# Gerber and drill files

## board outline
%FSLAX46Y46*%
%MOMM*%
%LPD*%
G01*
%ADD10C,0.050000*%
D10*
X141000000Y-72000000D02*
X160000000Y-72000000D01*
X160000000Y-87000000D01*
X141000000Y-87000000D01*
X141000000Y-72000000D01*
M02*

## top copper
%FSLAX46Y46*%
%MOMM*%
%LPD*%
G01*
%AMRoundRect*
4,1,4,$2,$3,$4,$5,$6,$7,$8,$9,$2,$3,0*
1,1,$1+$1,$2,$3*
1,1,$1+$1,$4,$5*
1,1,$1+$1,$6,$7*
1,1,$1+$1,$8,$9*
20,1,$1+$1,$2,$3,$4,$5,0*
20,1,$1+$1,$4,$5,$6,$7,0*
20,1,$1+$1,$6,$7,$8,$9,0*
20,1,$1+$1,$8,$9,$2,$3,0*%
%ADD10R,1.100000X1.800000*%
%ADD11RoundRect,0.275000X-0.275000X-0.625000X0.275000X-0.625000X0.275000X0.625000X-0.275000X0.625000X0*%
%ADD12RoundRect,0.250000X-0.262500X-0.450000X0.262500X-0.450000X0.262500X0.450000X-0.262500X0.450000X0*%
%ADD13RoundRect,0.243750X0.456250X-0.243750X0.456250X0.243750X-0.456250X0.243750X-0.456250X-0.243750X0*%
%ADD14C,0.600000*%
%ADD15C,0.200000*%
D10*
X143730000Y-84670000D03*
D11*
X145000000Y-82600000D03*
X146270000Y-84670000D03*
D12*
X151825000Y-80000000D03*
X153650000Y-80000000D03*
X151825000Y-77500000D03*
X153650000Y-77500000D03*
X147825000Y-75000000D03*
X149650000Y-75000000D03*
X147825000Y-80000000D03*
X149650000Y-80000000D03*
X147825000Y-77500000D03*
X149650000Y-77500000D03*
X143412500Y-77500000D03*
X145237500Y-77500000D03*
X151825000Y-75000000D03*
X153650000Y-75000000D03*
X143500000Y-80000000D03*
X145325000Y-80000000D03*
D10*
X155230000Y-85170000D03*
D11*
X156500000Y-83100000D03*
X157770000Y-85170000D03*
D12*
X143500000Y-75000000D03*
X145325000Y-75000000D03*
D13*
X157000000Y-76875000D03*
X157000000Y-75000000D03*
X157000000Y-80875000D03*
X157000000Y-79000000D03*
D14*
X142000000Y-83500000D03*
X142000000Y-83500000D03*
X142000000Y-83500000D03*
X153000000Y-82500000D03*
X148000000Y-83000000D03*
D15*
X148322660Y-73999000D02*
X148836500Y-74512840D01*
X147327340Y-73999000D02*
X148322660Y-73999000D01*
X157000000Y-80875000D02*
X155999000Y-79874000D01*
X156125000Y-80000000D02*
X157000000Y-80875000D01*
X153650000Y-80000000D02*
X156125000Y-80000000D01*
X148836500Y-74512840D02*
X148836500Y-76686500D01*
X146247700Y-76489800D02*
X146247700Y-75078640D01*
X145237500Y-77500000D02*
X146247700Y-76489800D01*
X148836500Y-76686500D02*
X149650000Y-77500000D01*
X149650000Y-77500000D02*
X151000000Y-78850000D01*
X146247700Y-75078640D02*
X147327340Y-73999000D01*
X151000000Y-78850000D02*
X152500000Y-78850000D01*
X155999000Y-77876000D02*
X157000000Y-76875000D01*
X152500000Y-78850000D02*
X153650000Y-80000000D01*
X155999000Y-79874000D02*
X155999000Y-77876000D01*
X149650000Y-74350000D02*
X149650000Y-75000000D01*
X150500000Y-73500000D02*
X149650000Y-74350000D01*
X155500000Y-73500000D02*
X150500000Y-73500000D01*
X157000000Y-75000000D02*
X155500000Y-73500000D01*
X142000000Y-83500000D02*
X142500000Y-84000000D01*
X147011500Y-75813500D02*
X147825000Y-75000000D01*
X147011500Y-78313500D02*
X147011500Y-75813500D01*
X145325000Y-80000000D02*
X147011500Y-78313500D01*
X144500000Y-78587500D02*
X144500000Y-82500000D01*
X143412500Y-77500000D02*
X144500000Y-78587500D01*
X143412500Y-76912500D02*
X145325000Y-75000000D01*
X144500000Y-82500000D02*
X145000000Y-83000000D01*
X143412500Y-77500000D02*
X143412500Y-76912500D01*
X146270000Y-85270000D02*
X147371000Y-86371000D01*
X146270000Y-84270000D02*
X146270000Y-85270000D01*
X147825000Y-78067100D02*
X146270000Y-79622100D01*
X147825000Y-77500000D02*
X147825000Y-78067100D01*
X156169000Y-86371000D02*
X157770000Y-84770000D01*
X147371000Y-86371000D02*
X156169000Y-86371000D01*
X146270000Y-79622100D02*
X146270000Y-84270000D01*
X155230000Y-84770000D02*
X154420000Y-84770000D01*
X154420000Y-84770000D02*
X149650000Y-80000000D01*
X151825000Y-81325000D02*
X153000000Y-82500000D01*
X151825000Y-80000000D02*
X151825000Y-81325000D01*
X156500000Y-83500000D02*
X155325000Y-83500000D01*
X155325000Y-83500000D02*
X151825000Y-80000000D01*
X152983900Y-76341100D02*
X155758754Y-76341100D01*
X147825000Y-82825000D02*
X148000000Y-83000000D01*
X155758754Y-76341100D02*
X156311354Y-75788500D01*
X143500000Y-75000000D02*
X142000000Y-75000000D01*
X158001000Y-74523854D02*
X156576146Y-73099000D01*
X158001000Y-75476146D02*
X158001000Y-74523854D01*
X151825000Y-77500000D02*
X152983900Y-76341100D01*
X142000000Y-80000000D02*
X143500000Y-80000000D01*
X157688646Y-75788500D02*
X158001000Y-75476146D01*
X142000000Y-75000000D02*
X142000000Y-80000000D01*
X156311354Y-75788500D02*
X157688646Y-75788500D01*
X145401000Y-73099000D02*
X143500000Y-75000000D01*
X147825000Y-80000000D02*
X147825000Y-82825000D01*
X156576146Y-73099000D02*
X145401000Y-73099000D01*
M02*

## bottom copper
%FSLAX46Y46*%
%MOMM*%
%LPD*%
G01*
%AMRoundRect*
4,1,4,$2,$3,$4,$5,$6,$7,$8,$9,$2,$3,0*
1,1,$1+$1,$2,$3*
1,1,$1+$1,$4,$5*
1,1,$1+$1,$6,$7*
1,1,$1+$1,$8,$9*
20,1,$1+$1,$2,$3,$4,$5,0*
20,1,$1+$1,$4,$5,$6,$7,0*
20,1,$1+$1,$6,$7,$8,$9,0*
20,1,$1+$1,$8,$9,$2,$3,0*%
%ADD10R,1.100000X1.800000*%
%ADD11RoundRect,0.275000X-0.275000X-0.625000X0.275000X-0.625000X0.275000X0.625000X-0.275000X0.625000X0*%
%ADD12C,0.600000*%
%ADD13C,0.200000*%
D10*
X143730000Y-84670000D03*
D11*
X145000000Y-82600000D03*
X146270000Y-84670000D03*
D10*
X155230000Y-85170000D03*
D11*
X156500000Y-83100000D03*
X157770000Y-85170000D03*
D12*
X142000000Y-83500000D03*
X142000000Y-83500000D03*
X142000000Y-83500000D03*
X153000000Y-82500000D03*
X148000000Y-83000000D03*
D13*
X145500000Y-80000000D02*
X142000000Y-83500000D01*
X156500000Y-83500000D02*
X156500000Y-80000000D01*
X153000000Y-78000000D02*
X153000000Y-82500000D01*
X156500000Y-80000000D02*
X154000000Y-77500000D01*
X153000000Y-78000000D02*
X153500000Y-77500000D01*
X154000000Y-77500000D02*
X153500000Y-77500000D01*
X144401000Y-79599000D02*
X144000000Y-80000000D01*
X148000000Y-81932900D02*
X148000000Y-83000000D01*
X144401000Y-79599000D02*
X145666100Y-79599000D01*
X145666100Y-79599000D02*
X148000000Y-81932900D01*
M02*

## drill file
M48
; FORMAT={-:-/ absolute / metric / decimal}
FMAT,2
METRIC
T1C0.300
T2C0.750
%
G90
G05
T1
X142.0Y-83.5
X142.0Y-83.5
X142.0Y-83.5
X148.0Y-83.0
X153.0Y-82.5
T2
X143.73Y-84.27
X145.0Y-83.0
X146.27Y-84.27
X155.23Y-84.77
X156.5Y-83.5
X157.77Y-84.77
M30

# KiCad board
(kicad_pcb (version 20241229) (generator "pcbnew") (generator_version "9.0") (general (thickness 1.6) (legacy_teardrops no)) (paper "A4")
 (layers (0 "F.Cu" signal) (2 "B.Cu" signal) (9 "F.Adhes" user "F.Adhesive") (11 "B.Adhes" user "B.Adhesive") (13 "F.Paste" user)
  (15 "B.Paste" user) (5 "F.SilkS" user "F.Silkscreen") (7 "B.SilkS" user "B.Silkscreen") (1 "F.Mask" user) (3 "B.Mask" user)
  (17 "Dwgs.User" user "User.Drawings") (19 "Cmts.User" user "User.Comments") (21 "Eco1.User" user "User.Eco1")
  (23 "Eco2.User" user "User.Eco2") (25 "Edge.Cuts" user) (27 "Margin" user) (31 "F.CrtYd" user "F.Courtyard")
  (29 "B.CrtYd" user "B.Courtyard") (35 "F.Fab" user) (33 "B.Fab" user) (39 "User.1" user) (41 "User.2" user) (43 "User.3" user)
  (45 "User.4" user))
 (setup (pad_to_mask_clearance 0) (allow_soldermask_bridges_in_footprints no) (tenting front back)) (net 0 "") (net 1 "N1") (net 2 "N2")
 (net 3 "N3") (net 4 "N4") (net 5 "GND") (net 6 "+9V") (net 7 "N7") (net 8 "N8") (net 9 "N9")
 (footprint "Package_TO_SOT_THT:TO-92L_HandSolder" (layer "F.Cu") (at 143.73 84.27)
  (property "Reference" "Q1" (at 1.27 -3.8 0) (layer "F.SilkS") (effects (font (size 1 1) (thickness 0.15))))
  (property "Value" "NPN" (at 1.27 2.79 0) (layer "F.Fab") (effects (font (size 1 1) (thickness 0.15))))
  (pad "1" thru_hole rect (at 0 0) (size 1.1 1.8) (drill 0.75 (offset 0 0.4)) (layers "*.Cu" "*.Mask") (remove_unused_layers no)
   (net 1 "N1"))
  (pad "2" thru_hole roundrect (at 1.27 -1.27) (size 1.1 1.8) (drill 0.75 (offset 0 -0.4)) (layers "*.Cu" "*.Mask")
   (remove_unused_layers no) (roundrect_rratio 0.25) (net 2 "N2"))
  (pad "3" thru_hole roundrect (at 2.54 0) (size 1.1 1.8) (drill 0.75 (offset 0 0.4)) (layers "*.Cu" "*.Mask") (remove_unused_layers no)
   (roundrect_rratio 0.25) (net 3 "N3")))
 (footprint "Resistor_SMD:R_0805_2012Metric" (layer "F.Cu") (at 152.7375 80)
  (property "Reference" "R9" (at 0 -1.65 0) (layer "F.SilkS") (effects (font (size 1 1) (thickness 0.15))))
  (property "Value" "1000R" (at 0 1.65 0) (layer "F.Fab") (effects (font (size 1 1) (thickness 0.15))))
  (pad "1" smd roundrect (at -0.9125 0) (size 1.025 1.4) (layers "F.Cu" "F.Mask" "F.Paste") (roundrect_rratio 0.243902) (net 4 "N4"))
  (pad "2" smd roundrect (at 0.9125 0) (size 1.025 1.4) (layers "F.Cu" "F.Mask" "F.Paste") (roundrect_rratio 0.243902) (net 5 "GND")))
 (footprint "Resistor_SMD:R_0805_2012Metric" (layer "F.Cu") (at 152.7375 77.5)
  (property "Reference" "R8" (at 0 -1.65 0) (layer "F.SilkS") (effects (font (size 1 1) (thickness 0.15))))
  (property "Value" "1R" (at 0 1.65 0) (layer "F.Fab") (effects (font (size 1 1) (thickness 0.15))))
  (pad "1" smd roundrect (at -0.9125 0) (size 1.025 1.4) (layers "F.Cu" "F.Mask" "F.Paste") (roundrect_rratio 0.243902) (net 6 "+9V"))
  (pad "2" smd roundrect (at 0.9125 0) (size 1.025 1.4) (layers "F.Cu" "F.Mask" "F.Paste") (roundrect_rratio 0.243902) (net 4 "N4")))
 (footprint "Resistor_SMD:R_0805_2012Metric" (layer "F.Cu") (at 148.7375 75)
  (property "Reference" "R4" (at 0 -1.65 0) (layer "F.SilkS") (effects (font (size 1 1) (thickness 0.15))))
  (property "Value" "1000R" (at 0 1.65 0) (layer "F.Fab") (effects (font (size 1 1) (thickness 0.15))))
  (pad "1" smd roundrect (at -0.9125 0) (size 1.025 1.4) (layers "F.Cu" "F.Mask" "F.Paste") (roundrect_rratio 0.243902) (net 1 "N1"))
  (pad "2" smd roundrect (at 0.9125 0) (size 1.025 1.4) (layers "F.Cu" "F.Mask" "F.Paste") (roundrect_rratio 0.243902) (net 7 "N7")))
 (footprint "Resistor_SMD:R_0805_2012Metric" (layer "F.Cu") (at 148.7375 80)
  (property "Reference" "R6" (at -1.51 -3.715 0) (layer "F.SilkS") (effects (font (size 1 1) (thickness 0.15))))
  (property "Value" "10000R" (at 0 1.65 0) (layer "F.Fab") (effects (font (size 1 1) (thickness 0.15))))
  (pad "1" smd roundrect (at -0.9125 0) (size 1.025 1.4) (layers "F.Cu" "F.Mask" "F.Paste") (roundrect_rratio 0.243902) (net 6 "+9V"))
  (pad "2" smd roundrect (at 0.9125 0) (size 1.025 1.4) (layers "F.Cu" "F.Mask" "F.Paste") (roundrect_rratio 0.243902) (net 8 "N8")))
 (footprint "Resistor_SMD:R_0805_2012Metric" (layer "F.Cu") (at 148.7375 77.5)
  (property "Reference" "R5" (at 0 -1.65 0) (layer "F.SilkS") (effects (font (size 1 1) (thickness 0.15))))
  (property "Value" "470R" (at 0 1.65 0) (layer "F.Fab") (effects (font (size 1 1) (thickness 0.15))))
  (pad "1" smd roundrect (at -0.9125 0) (size 1.025 1.4) (layers "F.Cu" "F.Mask" "F.Paste") (roundrect_rratio 0.243902) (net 3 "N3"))
  (pad "2" smd roundrect (at 0.9125 0) (size 1.025 1.4) (layers "F.Cu" "F.Mask" "F.Paste") (roundrect_rratio 0.243902) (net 5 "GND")))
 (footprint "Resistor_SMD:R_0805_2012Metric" (layer "F.Cu") (at 144.325 77.5)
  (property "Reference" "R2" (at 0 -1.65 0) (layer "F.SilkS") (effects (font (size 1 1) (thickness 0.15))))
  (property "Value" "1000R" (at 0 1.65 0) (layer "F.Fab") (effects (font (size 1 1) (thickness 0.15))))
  (pad "1" smd roundrect (at -0.9125 0) (size 1.025 1.4) (layers "F.Cu" "F.Mask" "F.Paste") (roundrect_rratio 0.243902) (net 2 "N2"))
  (pad "2" smd roundrect (at 0.9125 0) (size 1.025 1.4) (layers "F.Cu" "F.Mask" "F.Paste") (roundrect_rratio 0.243902) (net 5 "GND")))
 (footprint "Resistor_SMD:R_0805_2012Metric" (layer "F.Cu") (at 152.7375 75)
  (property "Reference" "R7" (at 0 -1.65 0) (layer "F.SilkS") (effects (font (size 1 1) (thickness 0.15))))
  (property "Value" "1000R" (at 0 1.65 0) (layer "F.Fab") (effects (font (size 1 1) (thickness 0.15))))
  (pad "1" smd roundrect (at -0.9125 0) (size 1.025 1.4) (layers "F.Cu" "F.Mask" "F.Paste") (roundrect_rratio 0.243902) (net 8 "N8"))
  (pad "2" smd roundrect (at 0.9125 0) (size 1.025 1.4) (layers "F.Cu" "F.Mask" "F.Paste") (roundrect_rratio 0.243902) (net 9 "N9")))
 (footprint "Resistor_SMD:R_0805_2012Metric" (layer "F.Cu") (at 144.4125 80)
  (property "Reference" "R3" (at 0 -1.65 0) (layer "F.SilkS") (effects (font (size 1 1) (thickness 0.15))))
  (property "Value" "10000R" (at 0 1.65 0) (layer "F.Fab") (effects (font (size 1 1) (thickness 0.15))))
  (pad "1" smd roundrect (at -0.9125 0) (size 1.025 1.4) (layers "F.Cu" "F.Mask" "F.Paste") (roundrect_rratio 0.243902) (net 6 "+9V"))
  (pad "2" smd roundrect (at 0.9125 0) (size 1.025 1.4) (layers "F.Cu" "F.Mask" "F.Paste") (roundrect_rratio 0.243902) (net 1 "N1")))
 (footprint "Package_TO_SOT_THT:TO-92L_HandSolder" (layer "F.Cu") (at 155.23 84.77)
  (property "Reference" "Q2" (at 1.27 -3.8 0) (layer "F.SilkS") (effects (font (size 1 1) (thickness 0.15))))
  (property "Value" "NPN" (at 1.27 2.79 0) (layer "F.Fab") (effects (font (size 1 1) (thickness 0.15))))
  (pad "1" thru_hole rect (at 0 0) (size 1.1 1.8) (drill 0.75 (offset 0 0.4)) (layers "*.Cu" "*.Mask") (remove_unused_layers no)
   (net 8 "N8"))
  (pad "2" thru_hole roundrect (at 1.27 -1.27) (size 1.1 1.8) (drill 0.75 (offset 0 -0.4)) (layers "*.Cu" "*.Mask")
   (remove_unused_layers no) (roundrect_rratio 0.25) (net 4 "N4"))
  (pad "3" thru_hole roundrect (at 2.54 0) (size 1.1 1.8) (drill 0.75 (offset 0 0.4)) (layers "*.Cu" "*.Mask") (remove_unused_layers no)
   (roundrect_rratio 0.25) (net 3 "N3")))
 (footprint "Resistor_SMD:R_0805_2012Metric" (layer "F.Cu") (at 144.4125 75)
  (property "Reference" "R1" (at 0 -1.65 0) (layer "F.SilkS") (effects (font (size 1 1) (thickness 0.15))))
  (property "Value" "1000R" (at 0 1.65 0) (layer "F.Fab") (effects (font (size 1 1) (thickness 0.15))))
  (pad "1" smd roundrect (at -0.9125 0) (size 1.025 1.4) (layers "F.Cu" "F.Mask" "F.Paste") (roundrect_rratio 0.243902) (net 6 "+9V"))
  (pad "2" smd roundrect (at 0.9125 0) (size 1.025 1.4) (layers "F.Cu" "F.Mask" "F.Paste") (roundrect_rratio 0.243902) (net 2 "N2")))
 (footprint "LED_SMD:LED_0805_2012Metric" (layer "F.Cu") (at 157 75.9375 90)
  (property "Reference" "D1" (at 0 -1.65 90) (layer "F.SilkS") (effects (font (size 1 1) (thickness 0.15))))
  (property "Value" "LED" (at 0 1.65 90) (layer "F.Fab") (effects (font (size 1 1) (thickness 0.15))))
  (pad "1" smd roundrect (at -0.9375 0 90) (size 0.975 1.4) (layers "F.Cu" "F.Mask" "F.Paste") (roundrect_rratio 0.25) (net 5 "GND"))
  (pad "2" smd roundrect (at 0.9375 0 90) (size 0.975 1.4) (layers "F.Cu" "F.Mask" "F.Paste") (roundrect_rratio 0.25) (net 7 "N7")))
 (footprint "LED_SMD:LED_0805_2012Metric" (layer "F.Cu") (at 157 79.9375 90)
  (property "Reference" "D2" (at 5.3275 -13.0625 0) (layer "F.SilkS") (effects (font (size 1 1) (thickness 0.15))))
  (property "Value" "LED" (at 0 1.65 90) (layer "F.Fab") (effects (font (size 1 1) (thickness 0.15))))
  (pad "1" smd roundrect (at -0.9375 0 90) (size 0.975 1.4) (layers "F.Cu" "F.Mask" "F.Paste") (roundrect_rratio 0.25) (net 5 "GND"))
  (pad "2" smd roundrect (at 0.9375 0 90) (size 0.975 1.4) (layers "F.Cu" "F.Mask" "F.Paste") (roundrect_rratio 0.25) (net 9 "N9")))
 (gr_rect (start 141 72) (end 160 87) (stroke (width 0.05) (type solid)) (fill no) (layer "Edge.Cuts"))
 (segment (start 148.32266 73.999) (end 148.8365 74.51284) (width 0.2) (layer "F.Cu") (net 5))
 (segment (start 147.32734 73.999) (end 148.32266 73.999) (width 0.2) (layer "F.Cu") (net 5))
 (segment (start 157 80.875) (end 155.999 79.874) (width 0.2) (layer "F.Cu") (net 5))
 (segment (start 156.125 80) (end 157 80.875) (width 0.2) (layer "F.Cu") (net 5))
 (segment (start 153.65 80) (end 156.125 80) (width 0.2) (layer "F.Cu") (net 5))
 (segment (start 148.8365 74.51284) (end 148.8365 76.6865) (width 0.2) (layer "F.Cu") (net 5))
 (segment (start 146.2477 76.4898) (end 146.2477 75.07864) (width 0.2) (layer "F.Cu") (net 5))
 (segment (start 145.2375 77.5) (end 146.2477 76.4898) (width 0.2) (layer "F.Cu") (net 5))
 (segment (start 148.8365 76.6865) (end 149.65 77.5) (width 0.2) (layer "F.Cu") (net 5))
 (segment (start 149.65 77.5) (end 151 78.85) (width 0.2) (layer "F.Cu") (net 5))
 (segment (start 146.2477 75.07864) (end 147.32734 73.999) (width 0.2) (layer "F.Cu") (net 5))
 (segment (start 151 78.85) (end 152.5 78.85) (width 0.2) (layer "F.Cu") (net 5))
 (segment (start 155.999 77.876) (end 157 76.875) (width 0.2) (layer "F.Cu") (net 5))
 (segment (start 152.5 78.85) (end 153.65 80) (width 0.2) (layer "F.Cu") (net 5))
 (segment (start 155.999 79.874) (end 155.999 77.876) (width 0.2) (layer "F.Cu") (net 5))
 (segment (start 149.65 74.35) (end 149.65 75) (width 0.2) (layer "F.Cu") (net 7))
 (segment (start 150.5 73.5) (end 149.65 74.35) (width 0.2) (layer "F.Cu") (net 7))
 (segment (start 155.5 73.5) (end 150.5 73.5) (width 0.2) (layer "F.Cu") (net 7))
 (segment (start 157 75) (end 155.5 73.5) (width 0.2) (layer "F.Cu") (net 7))
 (segment (start 142 83.5) (end 142.5 84) (width 0.2) (layer "F.Cu") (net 1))
 (segment (start 147.0115 75.8135) (end 147.825 75) (width 0.2) (layer "F.Cu") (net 1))
 (segment (start 147.0115 78.3135) (end 147.0115 75.8135) (width 0.2) (layer "F.Cu") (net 1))
 (segment (start 145.325 80) (end 147.0115 78.3135) (width 0.2) (layer "F.Cu") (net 1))
 (via (at 142 83.5) (size 0.6) (drill 0.3) (layers "F.Cu" "B.Cu") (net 1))
 (via (at 142 83.5) (size 0.6) (drill 0.3) (layers "F.Cu" "B.Cu") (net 1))
 (via (at 142 83.5) (size 0.6) (drill 0.3) (layers "F.Cu" "B.Cu") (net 1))
 (segment (start 145.5 80) (end 142 83.5) (width 0.2) (layer "B.Cu") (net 1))
 (segment (start 144.5 78.5875) (end 144.5 82.5) (width 0.2) (layer "F.Cu") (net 2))
 (segment (start 143.4125 77.5) (end 144.5 78.5875) (width 0.2) (layer "F.Cu") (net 2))
 (segment (start 143.4125 76.9125) (end 145.325 75) (width 0.2) (layer "F.Cu") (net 2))
 (segment (start 144.5 82.5) (end 145 83) (width 0.2) (layer "F.Cu") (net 2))
 (segment (start 143.4125 77.5) (end 143.4125 76.9125) (width 0.2) (layer "F.Cu") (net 2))
 (segment (start 146.27 85.27) (end 147.371 86.371) (width 0.2) (layer "F.Cu") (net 3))
 (segment (start 146.27 84.27) (end 146.27 85.27) (width 0.2) (layer "F.Cu") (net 3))
 (segment (start 147.825 78.0671) (end 146.27 79.6221) (width 0.2) (layer "F.Cu") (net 3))
 (segment (start 147.825 77.5) (end 147.825 78.0671) (width 0.2) (layer "F.Cu") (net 3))
 (segment (start 156.169 86.371) (end 157.77 84.77) (width 0.2) (layer "F.Cu") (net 3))
 (segment (start 147.371 86.371) (end 156.169 86.371) (width 0.2) (layer "F.Cu") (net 3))
 (segment (start 146.27 79.6221) (end 146.27 84.27) (width 0.2) (layer "F.Cu") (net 3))
 (segment (start 155.23 84.77) (end 154.42 84.77) (width 0.2) (layer "F.Cu") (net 8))
 (segment (start 154.42 84.77) (end 149.65 80) (width 0.2) (layer "F.Cu") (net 8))
 (segment (start 151.825 81.325) (end 153 82.5) (width 0.2) (layer "F.Cu") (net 4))
 (segment (start 151.825 80) (end 151.825 81.325) (width 0.2) (layer "F.Cu") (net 4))
 (segment (start 156.5 83.5) (end 155.325 83.5) (width 0.2) (layer "F.Cu") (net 4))
 (segment (start 155.325 83.5) (end 151.825 80) (width 0.2) (layer "F.Cu") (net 4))
 (via (at 153 82.5) (size 0.6) (drill 0.3) (layers "F.Cu" "B.Cu") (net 4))
 (segment (start 156.5 83.5) (end 156.5 80) (width 0.2) (layer "B.Cu") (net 4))
 (segment (start 153 78) (end 153 82.5) (width 0.2) (layer "B.Cu") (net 4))
 (segment (start 156.5 80) (end 154 77.5) (width 0.2) (layer "B.Cu") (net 4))
 (segment (start 153 78) (end 153.5 77.5) (width 0.2) (layer "B.Cu") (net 4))
 (segment (start 154 77.5) (end 153.5 77.5) (width 0.2) (layer "B.Cu") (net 4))
 (segment (start 152.9839 76.3411) (end 155.758754 76.3411) (width 0.2) (layer "F.Cu") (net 6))
 (segment (start 147.825 82.825) (end 148 83) (width 0.2) (layer "F.Cu") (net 6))
 (segment (start 155.758754 76.3411) (end 156.311354 75.7885) (width 0.2) (layer "F.Cu") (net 6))
 (segment (start 143.5 75) (end 142 75) (width 0.2) (layer "F.Cu") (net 6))
 (segment (start 158.001 74.523854) (end 156.576146 73.099) (width 0.2) (layer "F.Cu") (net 6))
 (segment (start 158.001 75.476146) (end 158.001 74.523854) (width 0.2) (layer "F.Cu") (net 6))
 (segment (start 151.825 77.5) (end 152.9839 76.3411) (width 0.2) (layer "F.Cu") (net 6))
 (segment (start 142 80) (end 143.5 80) (width 0.2) (layer "F.Cu") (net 6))
 (segment (start 157.688646 75.7885) (end 158.001 75.476146) (width 0.2) (layer "F.Cu") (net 6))
 (segment (start 142 75) (end 142 80) (width 0.2) (layer "F.Cu") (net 6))
 (segment (start 156.311354 75.7885) (end 157.688646 75.7885) (width 0.2) (layer "F.Cu") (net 6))
 (segment (start 145.401 73.099) (end 143.5 75) (width 0.2) (layer "F.Cu") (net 6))
 (segment (start 147.825 80) (end 147.825 82.825) (width 0.2) (layer "F.Cu") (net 6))
 (segment (start 156.576146 73.099) (end 145.401 73.099) (width 0.2) (layer "F.Cu") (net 6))
 (via (at 148 83) (size 0.6) (drill 0.3) (layers "F.Cu" "B.Cu") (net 6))
 (segment (start 144.401 79.599) (end 144 80) (width 0.2) (layer "B.Cu") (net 6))
 (segment (start 148 81.9329) (end 148 83) (width 0.2) (layer "B.Cu") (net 6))
 (segment (start 144.401 79.599) (end 145.6661 79.599) (width 0.2) (layer "B.Cu") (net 6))
 (segment (start 145.6661 79.599) (end 148 81.9329) (width 0.2) (layer "B.Cu") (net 6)))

